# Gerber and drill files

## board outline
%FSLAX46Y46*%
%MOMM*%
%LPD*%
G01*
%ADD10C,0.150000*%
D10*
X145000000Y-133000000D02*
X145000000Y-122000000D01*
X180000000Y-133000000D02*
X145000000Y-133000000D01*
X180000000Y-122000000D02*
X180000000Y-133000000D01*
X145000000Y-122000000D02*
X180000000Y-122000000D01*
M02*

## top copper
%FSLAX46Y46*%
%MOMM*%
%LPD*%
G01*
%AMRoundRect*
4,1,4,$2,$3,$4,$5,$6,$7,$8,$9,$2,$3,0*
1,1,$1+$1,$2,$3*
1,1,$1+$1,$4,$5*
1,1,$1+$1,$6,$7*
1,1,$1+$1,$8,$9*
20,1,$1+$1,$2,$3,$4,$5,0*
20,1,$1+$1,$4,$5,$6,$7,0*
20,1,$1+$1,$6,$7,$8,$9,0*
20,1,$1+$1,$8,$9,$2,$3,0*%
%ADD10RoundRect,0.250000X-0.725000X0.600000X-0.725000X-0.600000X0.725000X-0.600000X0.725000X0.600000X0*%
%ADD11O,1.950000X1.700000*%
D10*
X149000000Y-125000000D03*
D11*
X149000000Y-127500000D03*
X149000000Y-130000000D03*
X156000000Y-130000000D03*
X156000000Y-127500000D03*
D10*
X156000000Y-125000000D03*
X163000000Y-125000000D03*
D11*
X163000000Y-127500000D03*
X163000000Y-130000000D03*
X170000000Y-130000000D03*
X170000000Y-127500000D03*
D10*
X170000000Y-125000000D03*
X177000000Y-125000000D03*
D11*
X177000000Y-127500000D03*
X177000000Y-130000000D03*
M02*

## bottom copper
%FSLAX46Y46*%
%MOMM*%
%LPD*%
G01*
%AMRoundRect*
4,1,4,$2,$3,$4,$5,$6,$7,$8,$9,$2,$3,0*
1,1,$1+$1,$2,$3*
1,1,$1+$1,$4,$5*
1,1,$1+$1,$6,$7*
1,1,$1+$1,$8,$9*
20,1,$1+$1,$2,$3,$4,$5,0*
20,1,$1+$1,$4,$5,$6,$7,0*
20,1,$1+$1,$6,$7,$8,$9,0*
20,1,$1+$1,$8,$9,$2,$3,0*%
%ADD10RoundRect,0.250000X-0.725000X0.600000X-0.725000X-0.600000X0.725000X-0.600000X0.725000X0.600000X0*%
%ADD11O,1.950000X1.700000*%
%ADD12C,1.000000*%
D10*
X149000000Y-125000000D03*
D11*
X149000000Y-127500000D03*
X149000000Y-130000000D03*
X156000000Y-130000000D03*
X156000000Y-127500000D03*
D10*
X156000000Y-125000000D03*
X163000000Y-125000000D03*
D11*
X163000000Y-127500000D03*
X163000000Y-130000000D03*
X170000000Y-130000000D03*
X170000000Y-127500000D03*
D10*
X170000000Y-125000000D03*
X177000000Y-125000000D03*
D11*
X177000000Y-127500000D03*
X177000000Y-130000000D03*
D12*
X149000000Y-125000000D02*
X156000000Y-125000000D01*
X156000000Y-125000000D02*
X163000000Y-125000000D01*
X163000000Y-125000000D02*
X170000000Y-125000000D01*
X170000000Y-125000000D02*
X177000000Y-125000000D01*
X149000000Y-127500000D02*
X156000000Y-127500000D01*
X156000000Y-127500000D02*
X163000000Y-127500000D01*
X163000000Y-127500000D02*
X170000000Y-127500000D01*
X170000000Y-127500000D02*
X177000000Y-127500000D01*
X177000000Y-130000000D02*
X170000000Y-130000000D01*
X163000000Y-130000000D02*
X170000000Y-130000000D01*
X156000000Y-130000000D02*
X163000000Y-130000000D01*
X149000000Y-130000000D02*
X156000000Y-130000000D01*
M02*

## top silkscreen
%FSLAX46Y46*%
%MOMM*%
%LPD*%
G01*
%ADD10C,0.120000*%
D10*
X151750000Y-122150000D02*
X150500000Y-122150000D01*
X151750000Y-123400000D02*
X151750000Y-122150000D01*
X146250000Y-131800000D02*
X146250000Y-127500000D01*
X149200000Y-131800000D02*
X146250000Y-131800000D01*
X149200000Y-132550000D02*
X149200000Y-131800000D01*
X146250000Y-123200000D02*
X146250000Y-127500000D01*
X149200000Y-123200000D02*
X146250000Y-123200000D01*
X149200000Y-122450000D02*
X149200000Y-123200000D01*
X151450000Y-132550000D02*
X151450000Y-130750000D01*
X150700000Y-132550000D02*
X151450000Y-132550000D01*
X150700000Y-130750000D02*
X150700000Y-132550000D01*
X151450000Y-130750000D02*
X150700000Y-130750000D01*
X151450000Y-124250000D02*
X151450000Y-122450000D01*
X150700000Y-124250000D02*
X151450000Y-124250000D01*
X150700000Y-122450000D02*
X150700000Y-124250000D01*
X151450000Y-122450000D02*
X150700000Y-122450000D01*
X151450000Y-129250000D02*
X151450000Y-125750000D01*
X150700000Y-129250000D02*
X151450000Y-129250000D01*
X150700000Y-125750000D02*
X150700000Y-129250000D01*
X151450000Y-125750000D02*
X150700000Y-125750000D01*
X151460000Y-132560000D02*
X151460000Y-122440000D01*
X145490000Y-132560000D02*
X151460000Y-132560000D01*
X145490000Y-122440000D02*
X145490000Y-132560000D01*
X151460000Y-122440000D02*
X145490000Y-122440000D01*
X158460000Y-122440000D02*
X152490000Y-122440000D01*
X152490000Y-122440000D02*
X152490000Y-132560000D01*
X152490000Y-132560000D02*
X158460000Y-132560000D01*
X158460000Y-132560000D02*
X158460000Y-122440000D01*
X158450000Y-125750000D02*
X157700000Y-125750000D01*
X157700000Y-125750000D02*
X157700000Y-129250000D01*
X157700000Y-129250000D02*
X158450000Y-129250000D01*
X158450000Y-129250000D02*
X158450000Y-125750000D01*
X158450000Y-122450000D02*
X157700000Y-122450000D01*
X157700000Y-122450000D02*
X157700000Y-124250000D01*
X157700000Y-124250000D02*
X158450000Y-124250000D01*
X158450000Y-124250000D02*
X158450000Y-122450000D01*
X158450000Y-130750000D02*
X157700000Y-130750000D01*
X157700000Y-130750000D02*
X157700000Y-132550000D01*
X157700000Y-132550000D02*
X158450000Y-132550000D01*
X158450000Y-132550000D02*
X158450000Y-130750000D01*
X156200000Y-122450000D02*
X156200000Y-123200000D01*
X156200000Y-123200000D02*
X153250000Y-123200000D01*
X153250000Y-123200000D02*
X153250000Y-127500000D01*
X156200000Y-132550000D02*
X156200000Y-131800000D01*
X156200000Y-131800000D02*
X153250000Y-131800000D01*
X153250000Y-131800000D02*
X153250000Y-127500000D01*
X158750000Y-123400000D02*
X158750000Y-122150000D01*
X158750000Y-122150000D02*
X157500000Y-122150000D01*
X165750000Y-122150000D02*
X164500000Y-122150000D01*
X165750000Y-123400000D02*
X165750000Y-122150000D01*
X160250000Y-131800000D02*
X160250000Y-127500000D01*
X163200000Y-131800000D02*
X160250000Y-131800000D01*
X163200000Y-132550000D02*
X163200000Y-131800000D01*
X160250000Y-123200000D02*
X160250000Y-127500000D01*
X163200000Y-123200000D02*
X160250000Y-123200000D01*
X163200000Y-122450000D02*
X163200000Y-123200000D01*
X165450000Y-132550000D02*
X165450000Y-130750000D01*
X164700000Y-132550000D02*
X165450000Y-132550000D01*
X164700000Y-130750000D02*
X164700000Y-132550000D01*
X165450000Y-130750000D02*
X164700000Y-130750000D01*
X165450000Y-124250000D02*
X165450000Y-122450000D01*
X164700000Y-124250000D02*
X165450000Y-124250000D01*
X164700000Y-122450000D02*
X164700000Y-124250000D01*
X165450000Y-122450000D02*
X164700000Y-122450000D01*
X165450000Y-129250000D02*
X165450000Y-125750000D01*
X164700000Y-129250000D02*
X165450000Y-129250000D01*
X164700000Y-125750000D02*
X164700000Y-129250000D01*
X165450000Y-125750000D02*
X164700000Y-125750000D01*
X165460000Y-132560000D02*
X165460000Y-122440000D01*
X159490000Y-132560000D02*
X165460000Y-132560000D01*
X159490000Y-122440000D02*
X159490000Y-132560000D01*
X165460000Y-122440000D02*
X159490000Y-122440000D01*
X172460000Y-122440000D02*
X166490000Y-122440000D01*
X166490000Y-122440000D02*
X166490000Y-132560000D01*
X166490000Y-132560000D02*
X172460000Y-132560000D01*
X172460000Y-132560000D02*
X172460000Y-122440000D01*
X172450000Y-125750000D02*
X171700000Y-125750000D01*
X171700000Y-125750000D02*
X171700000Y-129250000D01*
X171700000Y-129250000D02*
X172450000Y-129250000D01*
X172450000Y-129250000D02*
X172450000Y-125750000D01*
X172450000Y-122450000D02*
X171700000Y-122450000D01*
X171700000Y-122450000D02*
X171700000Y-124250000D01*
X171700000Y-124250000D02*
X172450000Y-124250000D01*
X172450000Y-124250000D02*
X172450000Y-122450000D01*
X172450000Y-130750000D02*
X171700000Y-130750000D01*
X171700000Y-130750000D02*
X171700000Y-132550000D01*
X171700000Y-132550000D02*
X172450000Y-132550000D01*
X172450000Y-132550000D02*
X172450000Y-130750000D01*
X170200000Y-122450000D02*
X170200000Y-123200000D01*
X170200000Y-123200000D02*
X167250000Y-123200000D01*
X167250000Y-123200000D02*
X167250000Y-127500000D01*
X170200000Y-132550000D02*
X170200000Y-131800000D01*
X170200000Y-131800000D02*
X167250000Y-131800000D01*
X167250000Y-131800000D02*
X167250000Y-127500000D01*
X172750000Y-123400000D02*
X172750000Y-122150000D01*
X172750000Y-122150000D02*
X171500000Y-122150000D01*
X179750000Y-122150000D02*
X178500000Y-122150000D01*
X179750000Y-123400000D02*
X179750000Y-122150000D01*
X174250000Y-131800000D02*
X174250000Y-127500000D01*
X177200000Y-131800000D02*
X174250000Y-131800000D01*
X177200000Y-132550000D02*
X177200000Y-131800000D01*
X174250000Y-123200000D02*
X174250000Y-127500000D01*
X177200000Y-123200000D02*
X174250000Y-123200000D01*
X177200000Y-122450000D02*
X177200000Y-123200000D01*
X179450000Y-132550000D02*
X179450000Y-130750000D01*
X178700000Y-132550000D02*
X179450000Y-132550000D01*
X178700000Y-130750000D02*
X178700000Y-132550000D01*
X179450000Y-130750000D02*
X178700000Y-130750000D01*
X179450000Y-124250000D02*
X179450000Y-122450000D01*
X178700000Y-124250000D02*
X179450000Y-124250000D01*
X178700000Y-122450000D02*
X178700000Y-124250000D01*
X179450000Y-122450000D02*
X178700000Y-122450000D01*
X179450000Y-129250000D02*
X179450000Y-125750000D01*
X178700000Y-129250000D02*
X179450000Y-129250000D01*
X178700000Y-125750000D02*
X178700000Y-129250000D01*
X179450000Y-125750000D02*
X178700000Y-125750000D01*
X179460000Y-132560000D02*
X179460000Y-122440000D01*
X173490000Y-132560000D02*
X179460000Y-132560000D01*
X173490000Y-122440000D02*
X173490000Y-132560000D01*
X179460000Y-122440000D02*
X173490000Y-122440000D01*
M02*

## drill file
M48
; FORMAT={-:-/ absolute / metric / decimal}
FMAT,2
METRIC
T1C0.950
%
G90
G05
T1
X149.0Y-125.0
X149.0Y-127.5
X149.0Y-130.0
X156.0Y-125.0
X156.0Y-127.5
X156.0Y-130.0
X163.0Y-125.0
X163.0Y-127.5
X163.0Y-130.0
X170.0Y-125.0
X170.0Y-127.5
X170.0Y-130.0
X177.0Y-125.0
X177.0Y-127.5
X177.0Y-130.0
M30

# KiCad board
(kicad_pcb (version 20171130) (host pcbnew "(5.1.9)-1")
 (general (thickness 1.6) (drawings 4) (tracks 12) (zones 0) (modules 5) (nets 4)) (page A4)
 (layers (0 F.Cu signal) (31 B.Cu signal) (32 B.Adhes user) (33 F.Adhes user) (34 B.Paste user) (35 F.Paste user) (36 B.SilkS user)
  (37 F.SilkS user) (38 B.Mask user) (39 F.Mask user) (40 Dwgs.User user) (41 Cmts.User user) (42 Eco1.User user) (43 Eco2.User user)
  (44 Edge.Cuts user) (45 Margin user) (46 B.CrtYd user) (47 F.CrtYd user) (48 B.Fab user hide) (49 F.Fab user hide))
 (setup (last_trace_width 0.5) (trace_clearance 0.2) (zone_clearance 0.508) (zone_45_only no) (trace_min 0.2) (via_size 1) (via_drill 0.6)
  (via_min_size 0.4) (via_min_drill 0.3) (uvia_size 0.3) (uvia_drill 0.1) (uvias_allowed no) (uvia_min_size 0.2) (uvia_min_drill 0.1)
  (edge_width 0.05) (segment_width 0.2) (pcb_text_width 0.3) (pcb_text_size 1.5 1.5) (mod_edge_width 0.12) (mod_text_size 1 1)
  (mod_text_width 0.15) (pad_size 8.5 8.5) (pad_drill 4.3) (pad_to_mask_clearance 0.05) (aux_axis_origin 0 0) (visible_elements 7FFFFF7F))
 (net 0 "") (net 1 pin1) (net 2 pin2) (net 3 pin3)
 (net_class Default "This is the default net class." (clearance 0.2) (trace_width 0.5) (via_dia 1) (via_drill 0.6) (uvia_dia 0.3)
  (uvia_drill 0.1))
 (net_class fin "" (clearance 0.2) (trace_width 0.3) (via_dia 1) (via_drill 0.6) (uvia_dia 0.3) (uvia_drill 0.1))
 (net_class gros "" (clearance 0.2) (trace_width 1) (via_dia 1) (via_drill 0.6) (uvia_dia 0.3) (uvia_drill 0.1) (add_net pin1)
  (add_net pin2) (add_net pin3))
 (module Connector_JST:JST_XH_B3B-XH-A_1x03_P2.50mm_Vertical (layer F.Cu) (at 149 125 270)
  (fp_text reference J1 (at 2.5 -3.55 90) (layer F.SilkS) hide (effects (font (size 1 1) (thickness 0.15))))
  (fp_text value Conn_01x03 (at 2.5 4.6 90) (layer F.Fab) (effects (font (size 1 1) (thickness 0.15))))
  (fp_line (start -2.85 -2.75) (end -2.85 -1.5) (layer F.SilkS) (width 0.12))
  (fp_line (start -1.6 -2.75) (end -2.85 -2.75) (layer F.SilkS) (width 0.12))
  (fp_line (start 6.8 2.75) (end 2.5 2.75) (layer F.SilkS) (width 0.12))
  (fp_line (start 6.8 -0.2) (end 6.8 2.75) (layer F.SilkS) (width 0.12))
  (fp_line (start 7.55 -0.2) (end 6.8 -0.2) (layer F.SilkS) (width 0.12))
  (fp_line (start -1.8 2.75) (end 2.5 2.75) (layer F.SilkS) (width 0.12))
  (fp_line (start -1.8 -0.2) (end -1.8 2.75) (layer F.SilkS) (width 0.12))
  (fp_line (start -2.55 -0.2) (end -1.8 -0.2) (layer F.SilkS) (width 0.12))
  (fp_line (start 7.55 -2.45) (end 5.75 -2.45) (layer F.SilkS) (width 0.12))
  (fp_line (start 7.55 -1.7) (end 7.55 -2.45) (layer F.SilkS) (width 0.12))
  (fp_line (start 5.75 -1.7) (end 7.55 -1.7) (layer F.SilkS) (width 0.12))
  (fp_line (start 5.75 -2.45) (end 5.75 -1.7) (layer F.SilkS) (width 0.12))
  (fp_line (start -0.75 -2.45) (end -2.55 -2.45) (layer F.SilkS) (width 0.12))
  (fp_line (start -0.75 -1.7) (end -0.75 -2.45) (layer F.SilkS) (width 0.12))
  (fp_line (start -2.55 -1.7) (end -0.75 -1.7) (layer F.SilkS) (width 0.12))
  (fp_line (start -2.55 -2.45) (end -2.55 -1.7) (layer F.SilkS) (width 0.12))
  (fp_line (start 4.25 -2.45) (end 0.75 -2.45) (layer F.SilkS) (width 0.12))
  (fp_line (start 4.25 -1.7) (end 4.25 -2.45) (layer F.SilkS) (width 0.12))
  (fp_line (start 0.75 -1.7) (end 4.25 -1.7) (layer F.SilkS) (width 0.12))
  (fp_line (start 0.75 -2.45) (end 0.75 -1.7) (layer F.SilkS) (width 0.12))
  (fp_line (start 7.56 -2.46) (end -2.56 -2.46) (layer F.SilkS) (width 0.12))
  (fp_line (start 7.56 3.51) (end 7.56 -2.46) (layer F.SilkS) (width 0.12))
  (fp_line (start -2.56 3.51) (end 7.56 3.51) (layer F.SilkS) (width 0.12))
  (fp_line (start -2.56 -2.46) (end -2.56 3.51) (layer F.SilkS) (width 0.12))
  (pad 1 thru_hole roundrect (at 0 0 270) (size 1.7 1.95) (drill 0.95) (layers *.Cu *.Mask) (roundrect_rratio 0.147059) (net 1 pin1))
  (pad 2 thru_hole oval (at 2.5 0 270) (size 1.7 1.95) (drill 0.95) (layers *.Cu *.Mask) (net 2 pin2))
  (pad 3 thru_hole oval (at 5 0 270) (size 1.7 1.95) (drill 0.95) (layers *.Cu *.Mask) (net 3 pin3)))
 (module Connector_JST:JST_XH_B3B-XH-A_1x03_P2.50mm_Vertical (layer F.Cu) (at 156 125 270)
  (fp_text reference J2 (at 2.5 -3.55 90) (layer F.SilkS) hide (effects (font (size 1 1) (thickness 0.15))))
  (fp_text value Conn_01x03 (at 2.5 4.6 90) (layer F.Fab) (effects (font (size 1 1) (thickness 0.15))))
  (fp_line (start -2.56 -2.46) (end -2.56 3.51) (layer F.SilkS) (width 0.12))
  (fp_line (start -2.56 3.51) (end 7.56 3.51) (layer F.SilkS) (width 0.12))
  (fp_line (start 7.56 3.51) (end 7.56 -2.46) (layer F.SilkS) (width 0.12))
  (fp_line (start 7.56 -2.46) (end -2.56 -2.46) (layer F.SilkS) (width 0.12))
  (fp_line (start 0.75 -2.45) (end 0.75 -1.7) (layer F.SilkS) (width 0.12))
  (fp_line (start 0.75 -1.7) (end 4.25 -1.7) (layer F.SilkS) (width 0.12))
  (fp_line (start 4.25 -1.7) (end 4.25 -2.45) (layer F.SilkS) (width 0.12))
  (fp_line (start 4.25 -2.45) (end 0.75 -2.45) (layer F.SilkS) (width 0.12))
  (fp_line (start -2.55 -2.45) (end -2.55 -1.7) (layer F.SilkS) (width 0.12))
  (fp_line (start -2.55 -1.7) (end -0.75 -1.7) (layer F.SilkS) (width 0.12))
  (fp_line (start -0.75 -1.7) (end -0.75 -2.45) (layer F.SilkS) (width 0.12))
  (fp_line (start -0.75 -2.45) (end -2.55 -2.45) (layer F.SilkS) (width 0.12))
  (fp_line (start 5.75 -2.45) (end 5.75 -1.7) (layer F.SilkS) (width 0.12))
  (fp_line (start 5.75 -1.7) (end 7.55 -1.7) (layer F.SilkS) (width 0.12))
  (fp_line (start 7.55 -1.7) (end 7.55 -2.45) (layer F.SilkS) (width 0.12))
  (fp_line (start 7.55 -2.45) (end 5.75 -2.45) (layer F.SilkS) (width 0.12))
  (fp_line (start -2.55 -0.2) (end -1.8 -0.2) (layer F.SilkS) (width 0.12))
  (fp_line (start -1.8 -0.2) (end -1.8 2.75) (layer F.SilkS) (width 0.12))
  (fp_line (start -1.8 2.75) (end 2.5 2.75) (layer F.SilkS) (width 0.12))
  (fp_line (start 7.55 -0.2) (end 6.8 -0.2) (layer F.SilkS) (width 0.12))
  (fp_line (start 6.8 -0.2) (end 6.8 2.75) (layer F.SilkS) (width 0.12))
  (fp_line (start 6.8 2.75) (end 2.5 2.75) (layer F.SilkS) (width 0.12))
  (fp_line (start -1.6 -2.75) (end -2.85 -2.75) (layer F.SilkS) (width 0.12))
  (fp_line (start -2.85 -2.75) (end -2.85 -1.5) (layer F.SilkS) (width 0.12))
  (pad 3 thru_hole oval (at 5 0 270) (size 1.7 1.95) (drill 0.95) (layers *.Cu *.Mask) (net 3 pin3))
  (pad 2 thru_hole oval (at 2.5 0 270) (size 1.7 1.95) (drill 0.95) (layers *.Cu *.Mask) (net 2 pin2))
  (pad 1 thru_hole roundrect (at 0 0 270) (size 1.7 1.95) (drill 0.95) (layers *.Cu *.Mask) (roundrect_rratio 0.147059) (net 1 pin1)))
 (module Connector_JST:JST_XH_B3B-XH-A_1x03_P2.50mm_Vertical (layer F.Cu) (at 163 125 270)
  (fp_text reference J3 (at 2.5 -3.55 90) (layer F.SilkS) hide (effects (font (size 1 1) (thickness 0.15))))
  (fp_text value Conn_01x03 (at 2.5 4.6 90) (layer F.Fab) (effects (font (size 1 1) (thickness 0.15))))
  (fp_line (start -2.85 -2.75) (end -2.85 -1.5) (layer F.SilkS) (width 0.12))
  (fp_line (start -1.6 -2.75) (end -2.85 -2.75) (layer F.SilkS) (width 0.12))
  (fp_line (start 6.8 2.75) (end 2.5 2.75) (layer F.SilkS) (width 0.12))
  (fp_line (start 6.8 -0.2) (end 6.8 2.75) (layer F.SilkS) (width 0.12))
  (fp_line (start 7.55 -0.2) (end 6.8 -0.2) (layer F.SilkS) (width 0.12))
  (fp_line (start -1.8 2.75) (end 2.5 2.75) (layer F.SilkS) (width 0.12))
  (fp_line (start -1.8 -0.2) (end -1.8 2.75) (layer F.SilkS) (width 0.12))
  (fp_line (start -2.55 -0.2) (end -1.8 -0.2) (layer F.SilkS) (width 0.12))
  (fp_line (start 7.55 -2.45) (end 5.75 -2.45) (layer F.SilkS) (width 0.12))
  (fp_line (start 7.55 -1.7) (end 7.55 -2.45) (layer F.SilkS) (width 0.12))
  (fp_line (start 5.75 -1.7) (end 7.55 -1.7) (layer F.SilkS) (width 0.12))
  (fp_line (start 5.75 -2.45) (end 5.75 -1.7) (layer F.SilkS) (width 0.12))
  (fp_line (start -0.75 -2.45) (end -2.55 -2.45) (layer F.SilkS) (width 0.12))
  (fp_line (start -0.75 -1.7) (end -0.75 -2.45) (layer F.SilkS) (width 0.12))
  (fp_line (start -2.55 -1.7) (end -0.75 -1.7) (layer F.SilkS) (width 0.12))
  (fp_line (start -2.55 -2.45) (end -2.55 -1.7) (layer F.SilkS) (width 0.12))
  (fp_line (start 4.25 -2.45) (end 0.75 -2.45) (layer F.SilkS) (width 0.12))
  (fp_line (start 4.25 -1.7) (end 4.25 -2.45) (layer F.SilkS) (width 0.12))
  (fp_line (start 0.75 -1.7) (end 4.25 -1.7) (layer F.SilkS) (width 0.12))
  (fp_line (start 0.75 -2.45) (end 0.75 -1.7) (layer F.SilkS) (width 0.12))
  (fp_line (start 7.56 -2.46) (end -2.56 -2.46) (layer F.SilkS) (width 0.12))
  (fp_line (start 7.56 3.51) (end 7.56 -2.46) (layer F.SilkS) (width 0.12))
  (fp_line (start -2.56 3.51) (end 7.56 3.51) (layer F.SilkS) (width 0.12))
  (fp_line (start -2.56 -2.46) (end -2.56 3.51) (layer F.SilkS) (width 0.12))
  (pad 1 thru_hole roundrect (at 0 0 270) (size 1.7 1.95) (drill 0.95) (layers *.Cu *.Mask) (roundrect_rratio 0.147059) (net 1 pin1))
  (pad 2 thru_hole oval (at 2.5 0 270) (size 1.7 1.95) (drill 0.95) (layers *.Cu *.Mask) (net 2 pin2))
  (pad 3 thru_hole oval (at 5 0 270) (size 1.7 1.95) (drill 0.95) (layers *.Cu *.Mask) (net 3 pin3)))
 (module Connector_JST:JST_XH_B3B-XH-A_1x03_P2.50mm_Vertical (layer F.Cu) (at 170 125 270)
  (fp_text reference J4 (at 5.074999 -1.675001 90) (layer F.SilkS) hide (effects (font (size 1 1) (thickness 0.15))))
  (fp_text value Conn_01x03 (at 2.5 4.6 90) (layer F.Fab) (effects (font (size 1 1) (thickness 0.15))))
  (fp_line (start -2.56 -2.46) (end -2.56 3.51) (layer F.SilkS) (width 0.12))
  (fp_line (start -2.56 3.51) (end 7.56 3.51) (layer F.SilkS) (width 0.12))
  (fp_line (start 7.56 3.51) (end 7.56 -2.46) (layer F.SilkS) (width 0.12))
  (fp_line (start 7.56 -2.46) (end -2.56 -2.46) (layer F.SilkS) (width 0.12))
  (fp_line (start 0.75 -2.45) (end 0.75 -1.7) (layer F.SilkS) (width 0.12))
  (fp_line (start 0.75 -1.7) (end 4.25 -1.7) (layer F.SilkS) (width 0.12))
  (fp_line (start 4.25 -1.7) (end 4.25 -2.45) (layer F.SilkS) (width 0.12))
  (fp_line (start 4.25 -2.45) (end 0.75 -2.45) (layer F.SilkS) (width 0.12))
  (fp_line (start -2.55 -2.45) (end -2.55 -1.7) (layer F.SilkS) (width 0.12))
  (fp_line (start -2.55 -1.7) (end -0.75 -1.7) (layer F.SilkS) (width 0.12))
  (fp_line (start -0.75 -1.7) (end -0.75 -2.45) (layer F.SilkS) (width 0.12))
  (fp_line (start -0.75 -2.45) (end -2.55 -2.45) (layer F.SilkS) (width 0.12))
  (fp_line (start 5.75 -2.45) (end 5.75 -1.7) (layer F.SilkS) (width 0.12))
  (fp_line (start 5.75 -1.7) (end 7.55 -1.7) (layer F.SilkS) (width 0.12))
  (fp_line (start 7.55 -1.7) (end 7.55 -2.45) (layer F.SilkS) (width 0.12))
  (fp_line (start 7.55 -2.45) (end 5.75 -2.45) (layer F.SilkS) (width 0.12))
  (fp_line (start -2.55 -0.2) (end -1.8 -0.2) (layer F.SilkS) (width 0.12))
  (fp_line (start -1.8 -0.2) (end -1.8 2.75) (layer F.SilkS) (width 0.12))
  (fp_line (start -1.8 2.75) (end 2.5 2.75) (layer F.SilkS) (width 0.12))
  (fp_line (start 7.55 -0.2) (end 6.8 -0.2) (layer F.SilkS) (width 0.12))
  (fp_line (start 6.8 -0.2) (end 6.8 2.75) (layer F.SilkS) (width 0.12))
  (fp_line (start 6.8 2.75) (end 2.5 2.75) (layer F.SilkS) (width 0.12))
  (fp_line (start -1.6 -2.75) (end -2.85 -2.75) (layer F.SilkS) (width 0.12))
  (fp_line (start -2.85 -2.75) (end -2.85 -1.5) (layer F.SilkS) (width 0.12))
  (pad 3 thru_hole oval (at 5 0 270) (size 1.7 1.95) (drill 0.95) (layers *.Cu *.Mask) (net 3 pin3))
  (pad 2 thru_hole oval (at 2.5 0 270) (size 1.7 1.95) (drill 0.95) (layers *.Cu *.Mask) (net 2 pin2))
  (pad 1 thru_hole roundrect (at 0 0 270) (size 1.7 1.95) (drill 0.95) (layers *.Cu *.Mask) (roundrect_rratio 0.147059) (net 1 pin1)))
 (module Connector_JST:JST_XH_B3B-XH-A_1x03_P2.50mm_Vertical (layer F.Cu) (at 177 125 270)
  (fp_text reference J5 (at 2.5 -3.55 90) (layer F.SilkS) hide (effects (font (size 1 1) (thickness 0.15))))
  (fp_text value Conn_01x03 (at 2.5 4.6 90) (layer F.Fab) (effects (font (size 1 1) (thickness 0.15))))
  (fp_line (start -2.85 -2.75) (end -2.85 -1.5) (layer F.SilkS) (width 0.12))
  (fp_line (start -1.6 -2.75) (end -2.85 -2.75) (layer F.SilkS) (width 0.12))
  (fp_line (start 6.8 2.75) (end 2.5 2.75) (layer F.SilkS) (width 0.12))
  (fp_line (start 6.8 -0.2) (end 6.8 2.75) (layer F.SilkS) (width 0.12))
  (fp_line (start 7.55 -0.2) (end 6.8 -0.2) (layer F.SilkS) (width 0.12))
  (fp_line (start -1.8 2.75) (end 2.5 2.75) (layer F.SilkS) (width 0.12))
  (fp_line (start -1.8 -0.2) (end -1.8 2.75) (layer F.SilkS) (width 0.12))
  (fp_line (start -2.55 -0.2) (end -1.8 -0.2) (layer F.SilkS) (width 0.12))
  (fp_line (start 7.55 -2.45) (end 5.75 -2.45) (layer F.SilkS) (width 0.12))
  (fp_line (start 7.55 -1.7) (end 7.55 -2.45) (layer F.SilkS) (width 0.12))
  (fp_line (start 5.75 -1.7) (end 7.55 -1.7) (layer F.SilkS) (width 0.12))
  (fp_line (start 5.75 -2.45) (end 5.75 -1.7) (layer F.SilkS) (width 0.12))
  (fp_line (start -0.75 -2.45) (end -2.55 -2.45) (layer F.SilkS) (width 0.12))
  (fp_line (start -0.75 -1.7) (end -0.75 -2.45) (layer F.SilkS) (width 0.12))
  (fp_line (start -2.55 -1.7) (end -0.75 -1.7) (layer F.SilkS) (width 0.12))
  (fp_line (start -2.55 -2.45) (end -2.55 -1.7) (layer F.SilkS) (width 0.12))
  (fp_line (start 4.25 -2.45) (end 0.75 -2.45) (layer F.SilkS) (width 0.12))
  (fp_line (start 4.25 -1.7) (end 4.25 -2.45) (layer F.SilkS) (width 0.12))
  (fp_line (start 0.75 -1.7) (end 4.25 -1.7) (layer F.SilkS) (width 0.12))
  (fp_line (start 0.75 -2.45) (end 0.75 -1.7) (layer F.SilkS) (width 0.12))
  (fp_line (start 7.56 -2.46) (end -2.56 -2.46) (layer F.SilkS) (width 0.12))
  (fp_line (start 7.56 3.51) (end 7.56 -2.46) (layer F.SilkS) (width 0.12))
  (fp_line (start -2.56 3.51) (end 7.56 3.51) (layer F.SilkS) (width 0.12))
  (fp_line (start -2.56 -2.46) (end -2.56 3.51) (layer F.SilkS) (width 0.12))
  (pad 1 thru_hole roundrect (at 0 0 270) (size 1.7 1.95) (drill 0.95) (layers *.Cu *.Mask) (roundrect_rratio 0.147059) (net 1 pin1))
  (pad 2 thru_hole oval (at 2.5 0 270) (size 1.7 1.95) (drill 0.95) (layers *.Cu *.Mask) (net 2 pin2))
  (pad 3 thru_hole oval (at 5 0 270) (size 1.7 1.95) (drill 0.95) (layers *.Cu *.Mask) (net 3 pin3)))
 (gr_line (start 145 133) (end 145 122) (layer Edge.Cuts) (width 0.15))
 (gr_line (start 180 133) (end 145 133) (layer Edge.Cuts) (width 0.15))
 (gr_line (start 180 122) (end 180 133) (layer Edge.Cuts) (width 0.15))
 (gr_line (start 145 122) (end 180 122) (layer Edge.Cuts) (width 0.15))
 (segment (start 149 125) (end 156 125) (width 1) (layer B.Cu) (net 1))
 (segment (start 156 125) (end 163 125) (width 1) (layer B.Cu) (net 1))
 (segment (start 163 125) (end 170 125) (width 1) (layer B.Cu) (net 1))
 (segment (start 170 125) (end 177 125) (width 1) (layer B.Cu) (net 1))
 (segment (start 149 127.5) (end 156 127.5) (width 1) (layer B.Cu) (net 2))
 (segment (start 156 127.5) (end 163 127.5) (width 1) (layer B.Cu) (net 2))
 (segment (start 163 127.5) (end 170 127.5) (width 1) (layer B.Cu) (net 2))
 (segment (start 170 127.5) (end 177 127.5) (width 1) (layer B.Cu) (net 2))
 (segment (start 177 130) (end 170 130) (width 1) (layer B.Cu) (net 3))
 (segment (start 163 130) (end 170 130) (width 1) (layer B.Cu) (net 3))
 (segment (start 156 130) (end 163 130) (width 1) (layer B.Cu) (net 3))
 (segment (start 149 130) (end 156 130) (width 1) (layer B.Cu) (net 3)))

